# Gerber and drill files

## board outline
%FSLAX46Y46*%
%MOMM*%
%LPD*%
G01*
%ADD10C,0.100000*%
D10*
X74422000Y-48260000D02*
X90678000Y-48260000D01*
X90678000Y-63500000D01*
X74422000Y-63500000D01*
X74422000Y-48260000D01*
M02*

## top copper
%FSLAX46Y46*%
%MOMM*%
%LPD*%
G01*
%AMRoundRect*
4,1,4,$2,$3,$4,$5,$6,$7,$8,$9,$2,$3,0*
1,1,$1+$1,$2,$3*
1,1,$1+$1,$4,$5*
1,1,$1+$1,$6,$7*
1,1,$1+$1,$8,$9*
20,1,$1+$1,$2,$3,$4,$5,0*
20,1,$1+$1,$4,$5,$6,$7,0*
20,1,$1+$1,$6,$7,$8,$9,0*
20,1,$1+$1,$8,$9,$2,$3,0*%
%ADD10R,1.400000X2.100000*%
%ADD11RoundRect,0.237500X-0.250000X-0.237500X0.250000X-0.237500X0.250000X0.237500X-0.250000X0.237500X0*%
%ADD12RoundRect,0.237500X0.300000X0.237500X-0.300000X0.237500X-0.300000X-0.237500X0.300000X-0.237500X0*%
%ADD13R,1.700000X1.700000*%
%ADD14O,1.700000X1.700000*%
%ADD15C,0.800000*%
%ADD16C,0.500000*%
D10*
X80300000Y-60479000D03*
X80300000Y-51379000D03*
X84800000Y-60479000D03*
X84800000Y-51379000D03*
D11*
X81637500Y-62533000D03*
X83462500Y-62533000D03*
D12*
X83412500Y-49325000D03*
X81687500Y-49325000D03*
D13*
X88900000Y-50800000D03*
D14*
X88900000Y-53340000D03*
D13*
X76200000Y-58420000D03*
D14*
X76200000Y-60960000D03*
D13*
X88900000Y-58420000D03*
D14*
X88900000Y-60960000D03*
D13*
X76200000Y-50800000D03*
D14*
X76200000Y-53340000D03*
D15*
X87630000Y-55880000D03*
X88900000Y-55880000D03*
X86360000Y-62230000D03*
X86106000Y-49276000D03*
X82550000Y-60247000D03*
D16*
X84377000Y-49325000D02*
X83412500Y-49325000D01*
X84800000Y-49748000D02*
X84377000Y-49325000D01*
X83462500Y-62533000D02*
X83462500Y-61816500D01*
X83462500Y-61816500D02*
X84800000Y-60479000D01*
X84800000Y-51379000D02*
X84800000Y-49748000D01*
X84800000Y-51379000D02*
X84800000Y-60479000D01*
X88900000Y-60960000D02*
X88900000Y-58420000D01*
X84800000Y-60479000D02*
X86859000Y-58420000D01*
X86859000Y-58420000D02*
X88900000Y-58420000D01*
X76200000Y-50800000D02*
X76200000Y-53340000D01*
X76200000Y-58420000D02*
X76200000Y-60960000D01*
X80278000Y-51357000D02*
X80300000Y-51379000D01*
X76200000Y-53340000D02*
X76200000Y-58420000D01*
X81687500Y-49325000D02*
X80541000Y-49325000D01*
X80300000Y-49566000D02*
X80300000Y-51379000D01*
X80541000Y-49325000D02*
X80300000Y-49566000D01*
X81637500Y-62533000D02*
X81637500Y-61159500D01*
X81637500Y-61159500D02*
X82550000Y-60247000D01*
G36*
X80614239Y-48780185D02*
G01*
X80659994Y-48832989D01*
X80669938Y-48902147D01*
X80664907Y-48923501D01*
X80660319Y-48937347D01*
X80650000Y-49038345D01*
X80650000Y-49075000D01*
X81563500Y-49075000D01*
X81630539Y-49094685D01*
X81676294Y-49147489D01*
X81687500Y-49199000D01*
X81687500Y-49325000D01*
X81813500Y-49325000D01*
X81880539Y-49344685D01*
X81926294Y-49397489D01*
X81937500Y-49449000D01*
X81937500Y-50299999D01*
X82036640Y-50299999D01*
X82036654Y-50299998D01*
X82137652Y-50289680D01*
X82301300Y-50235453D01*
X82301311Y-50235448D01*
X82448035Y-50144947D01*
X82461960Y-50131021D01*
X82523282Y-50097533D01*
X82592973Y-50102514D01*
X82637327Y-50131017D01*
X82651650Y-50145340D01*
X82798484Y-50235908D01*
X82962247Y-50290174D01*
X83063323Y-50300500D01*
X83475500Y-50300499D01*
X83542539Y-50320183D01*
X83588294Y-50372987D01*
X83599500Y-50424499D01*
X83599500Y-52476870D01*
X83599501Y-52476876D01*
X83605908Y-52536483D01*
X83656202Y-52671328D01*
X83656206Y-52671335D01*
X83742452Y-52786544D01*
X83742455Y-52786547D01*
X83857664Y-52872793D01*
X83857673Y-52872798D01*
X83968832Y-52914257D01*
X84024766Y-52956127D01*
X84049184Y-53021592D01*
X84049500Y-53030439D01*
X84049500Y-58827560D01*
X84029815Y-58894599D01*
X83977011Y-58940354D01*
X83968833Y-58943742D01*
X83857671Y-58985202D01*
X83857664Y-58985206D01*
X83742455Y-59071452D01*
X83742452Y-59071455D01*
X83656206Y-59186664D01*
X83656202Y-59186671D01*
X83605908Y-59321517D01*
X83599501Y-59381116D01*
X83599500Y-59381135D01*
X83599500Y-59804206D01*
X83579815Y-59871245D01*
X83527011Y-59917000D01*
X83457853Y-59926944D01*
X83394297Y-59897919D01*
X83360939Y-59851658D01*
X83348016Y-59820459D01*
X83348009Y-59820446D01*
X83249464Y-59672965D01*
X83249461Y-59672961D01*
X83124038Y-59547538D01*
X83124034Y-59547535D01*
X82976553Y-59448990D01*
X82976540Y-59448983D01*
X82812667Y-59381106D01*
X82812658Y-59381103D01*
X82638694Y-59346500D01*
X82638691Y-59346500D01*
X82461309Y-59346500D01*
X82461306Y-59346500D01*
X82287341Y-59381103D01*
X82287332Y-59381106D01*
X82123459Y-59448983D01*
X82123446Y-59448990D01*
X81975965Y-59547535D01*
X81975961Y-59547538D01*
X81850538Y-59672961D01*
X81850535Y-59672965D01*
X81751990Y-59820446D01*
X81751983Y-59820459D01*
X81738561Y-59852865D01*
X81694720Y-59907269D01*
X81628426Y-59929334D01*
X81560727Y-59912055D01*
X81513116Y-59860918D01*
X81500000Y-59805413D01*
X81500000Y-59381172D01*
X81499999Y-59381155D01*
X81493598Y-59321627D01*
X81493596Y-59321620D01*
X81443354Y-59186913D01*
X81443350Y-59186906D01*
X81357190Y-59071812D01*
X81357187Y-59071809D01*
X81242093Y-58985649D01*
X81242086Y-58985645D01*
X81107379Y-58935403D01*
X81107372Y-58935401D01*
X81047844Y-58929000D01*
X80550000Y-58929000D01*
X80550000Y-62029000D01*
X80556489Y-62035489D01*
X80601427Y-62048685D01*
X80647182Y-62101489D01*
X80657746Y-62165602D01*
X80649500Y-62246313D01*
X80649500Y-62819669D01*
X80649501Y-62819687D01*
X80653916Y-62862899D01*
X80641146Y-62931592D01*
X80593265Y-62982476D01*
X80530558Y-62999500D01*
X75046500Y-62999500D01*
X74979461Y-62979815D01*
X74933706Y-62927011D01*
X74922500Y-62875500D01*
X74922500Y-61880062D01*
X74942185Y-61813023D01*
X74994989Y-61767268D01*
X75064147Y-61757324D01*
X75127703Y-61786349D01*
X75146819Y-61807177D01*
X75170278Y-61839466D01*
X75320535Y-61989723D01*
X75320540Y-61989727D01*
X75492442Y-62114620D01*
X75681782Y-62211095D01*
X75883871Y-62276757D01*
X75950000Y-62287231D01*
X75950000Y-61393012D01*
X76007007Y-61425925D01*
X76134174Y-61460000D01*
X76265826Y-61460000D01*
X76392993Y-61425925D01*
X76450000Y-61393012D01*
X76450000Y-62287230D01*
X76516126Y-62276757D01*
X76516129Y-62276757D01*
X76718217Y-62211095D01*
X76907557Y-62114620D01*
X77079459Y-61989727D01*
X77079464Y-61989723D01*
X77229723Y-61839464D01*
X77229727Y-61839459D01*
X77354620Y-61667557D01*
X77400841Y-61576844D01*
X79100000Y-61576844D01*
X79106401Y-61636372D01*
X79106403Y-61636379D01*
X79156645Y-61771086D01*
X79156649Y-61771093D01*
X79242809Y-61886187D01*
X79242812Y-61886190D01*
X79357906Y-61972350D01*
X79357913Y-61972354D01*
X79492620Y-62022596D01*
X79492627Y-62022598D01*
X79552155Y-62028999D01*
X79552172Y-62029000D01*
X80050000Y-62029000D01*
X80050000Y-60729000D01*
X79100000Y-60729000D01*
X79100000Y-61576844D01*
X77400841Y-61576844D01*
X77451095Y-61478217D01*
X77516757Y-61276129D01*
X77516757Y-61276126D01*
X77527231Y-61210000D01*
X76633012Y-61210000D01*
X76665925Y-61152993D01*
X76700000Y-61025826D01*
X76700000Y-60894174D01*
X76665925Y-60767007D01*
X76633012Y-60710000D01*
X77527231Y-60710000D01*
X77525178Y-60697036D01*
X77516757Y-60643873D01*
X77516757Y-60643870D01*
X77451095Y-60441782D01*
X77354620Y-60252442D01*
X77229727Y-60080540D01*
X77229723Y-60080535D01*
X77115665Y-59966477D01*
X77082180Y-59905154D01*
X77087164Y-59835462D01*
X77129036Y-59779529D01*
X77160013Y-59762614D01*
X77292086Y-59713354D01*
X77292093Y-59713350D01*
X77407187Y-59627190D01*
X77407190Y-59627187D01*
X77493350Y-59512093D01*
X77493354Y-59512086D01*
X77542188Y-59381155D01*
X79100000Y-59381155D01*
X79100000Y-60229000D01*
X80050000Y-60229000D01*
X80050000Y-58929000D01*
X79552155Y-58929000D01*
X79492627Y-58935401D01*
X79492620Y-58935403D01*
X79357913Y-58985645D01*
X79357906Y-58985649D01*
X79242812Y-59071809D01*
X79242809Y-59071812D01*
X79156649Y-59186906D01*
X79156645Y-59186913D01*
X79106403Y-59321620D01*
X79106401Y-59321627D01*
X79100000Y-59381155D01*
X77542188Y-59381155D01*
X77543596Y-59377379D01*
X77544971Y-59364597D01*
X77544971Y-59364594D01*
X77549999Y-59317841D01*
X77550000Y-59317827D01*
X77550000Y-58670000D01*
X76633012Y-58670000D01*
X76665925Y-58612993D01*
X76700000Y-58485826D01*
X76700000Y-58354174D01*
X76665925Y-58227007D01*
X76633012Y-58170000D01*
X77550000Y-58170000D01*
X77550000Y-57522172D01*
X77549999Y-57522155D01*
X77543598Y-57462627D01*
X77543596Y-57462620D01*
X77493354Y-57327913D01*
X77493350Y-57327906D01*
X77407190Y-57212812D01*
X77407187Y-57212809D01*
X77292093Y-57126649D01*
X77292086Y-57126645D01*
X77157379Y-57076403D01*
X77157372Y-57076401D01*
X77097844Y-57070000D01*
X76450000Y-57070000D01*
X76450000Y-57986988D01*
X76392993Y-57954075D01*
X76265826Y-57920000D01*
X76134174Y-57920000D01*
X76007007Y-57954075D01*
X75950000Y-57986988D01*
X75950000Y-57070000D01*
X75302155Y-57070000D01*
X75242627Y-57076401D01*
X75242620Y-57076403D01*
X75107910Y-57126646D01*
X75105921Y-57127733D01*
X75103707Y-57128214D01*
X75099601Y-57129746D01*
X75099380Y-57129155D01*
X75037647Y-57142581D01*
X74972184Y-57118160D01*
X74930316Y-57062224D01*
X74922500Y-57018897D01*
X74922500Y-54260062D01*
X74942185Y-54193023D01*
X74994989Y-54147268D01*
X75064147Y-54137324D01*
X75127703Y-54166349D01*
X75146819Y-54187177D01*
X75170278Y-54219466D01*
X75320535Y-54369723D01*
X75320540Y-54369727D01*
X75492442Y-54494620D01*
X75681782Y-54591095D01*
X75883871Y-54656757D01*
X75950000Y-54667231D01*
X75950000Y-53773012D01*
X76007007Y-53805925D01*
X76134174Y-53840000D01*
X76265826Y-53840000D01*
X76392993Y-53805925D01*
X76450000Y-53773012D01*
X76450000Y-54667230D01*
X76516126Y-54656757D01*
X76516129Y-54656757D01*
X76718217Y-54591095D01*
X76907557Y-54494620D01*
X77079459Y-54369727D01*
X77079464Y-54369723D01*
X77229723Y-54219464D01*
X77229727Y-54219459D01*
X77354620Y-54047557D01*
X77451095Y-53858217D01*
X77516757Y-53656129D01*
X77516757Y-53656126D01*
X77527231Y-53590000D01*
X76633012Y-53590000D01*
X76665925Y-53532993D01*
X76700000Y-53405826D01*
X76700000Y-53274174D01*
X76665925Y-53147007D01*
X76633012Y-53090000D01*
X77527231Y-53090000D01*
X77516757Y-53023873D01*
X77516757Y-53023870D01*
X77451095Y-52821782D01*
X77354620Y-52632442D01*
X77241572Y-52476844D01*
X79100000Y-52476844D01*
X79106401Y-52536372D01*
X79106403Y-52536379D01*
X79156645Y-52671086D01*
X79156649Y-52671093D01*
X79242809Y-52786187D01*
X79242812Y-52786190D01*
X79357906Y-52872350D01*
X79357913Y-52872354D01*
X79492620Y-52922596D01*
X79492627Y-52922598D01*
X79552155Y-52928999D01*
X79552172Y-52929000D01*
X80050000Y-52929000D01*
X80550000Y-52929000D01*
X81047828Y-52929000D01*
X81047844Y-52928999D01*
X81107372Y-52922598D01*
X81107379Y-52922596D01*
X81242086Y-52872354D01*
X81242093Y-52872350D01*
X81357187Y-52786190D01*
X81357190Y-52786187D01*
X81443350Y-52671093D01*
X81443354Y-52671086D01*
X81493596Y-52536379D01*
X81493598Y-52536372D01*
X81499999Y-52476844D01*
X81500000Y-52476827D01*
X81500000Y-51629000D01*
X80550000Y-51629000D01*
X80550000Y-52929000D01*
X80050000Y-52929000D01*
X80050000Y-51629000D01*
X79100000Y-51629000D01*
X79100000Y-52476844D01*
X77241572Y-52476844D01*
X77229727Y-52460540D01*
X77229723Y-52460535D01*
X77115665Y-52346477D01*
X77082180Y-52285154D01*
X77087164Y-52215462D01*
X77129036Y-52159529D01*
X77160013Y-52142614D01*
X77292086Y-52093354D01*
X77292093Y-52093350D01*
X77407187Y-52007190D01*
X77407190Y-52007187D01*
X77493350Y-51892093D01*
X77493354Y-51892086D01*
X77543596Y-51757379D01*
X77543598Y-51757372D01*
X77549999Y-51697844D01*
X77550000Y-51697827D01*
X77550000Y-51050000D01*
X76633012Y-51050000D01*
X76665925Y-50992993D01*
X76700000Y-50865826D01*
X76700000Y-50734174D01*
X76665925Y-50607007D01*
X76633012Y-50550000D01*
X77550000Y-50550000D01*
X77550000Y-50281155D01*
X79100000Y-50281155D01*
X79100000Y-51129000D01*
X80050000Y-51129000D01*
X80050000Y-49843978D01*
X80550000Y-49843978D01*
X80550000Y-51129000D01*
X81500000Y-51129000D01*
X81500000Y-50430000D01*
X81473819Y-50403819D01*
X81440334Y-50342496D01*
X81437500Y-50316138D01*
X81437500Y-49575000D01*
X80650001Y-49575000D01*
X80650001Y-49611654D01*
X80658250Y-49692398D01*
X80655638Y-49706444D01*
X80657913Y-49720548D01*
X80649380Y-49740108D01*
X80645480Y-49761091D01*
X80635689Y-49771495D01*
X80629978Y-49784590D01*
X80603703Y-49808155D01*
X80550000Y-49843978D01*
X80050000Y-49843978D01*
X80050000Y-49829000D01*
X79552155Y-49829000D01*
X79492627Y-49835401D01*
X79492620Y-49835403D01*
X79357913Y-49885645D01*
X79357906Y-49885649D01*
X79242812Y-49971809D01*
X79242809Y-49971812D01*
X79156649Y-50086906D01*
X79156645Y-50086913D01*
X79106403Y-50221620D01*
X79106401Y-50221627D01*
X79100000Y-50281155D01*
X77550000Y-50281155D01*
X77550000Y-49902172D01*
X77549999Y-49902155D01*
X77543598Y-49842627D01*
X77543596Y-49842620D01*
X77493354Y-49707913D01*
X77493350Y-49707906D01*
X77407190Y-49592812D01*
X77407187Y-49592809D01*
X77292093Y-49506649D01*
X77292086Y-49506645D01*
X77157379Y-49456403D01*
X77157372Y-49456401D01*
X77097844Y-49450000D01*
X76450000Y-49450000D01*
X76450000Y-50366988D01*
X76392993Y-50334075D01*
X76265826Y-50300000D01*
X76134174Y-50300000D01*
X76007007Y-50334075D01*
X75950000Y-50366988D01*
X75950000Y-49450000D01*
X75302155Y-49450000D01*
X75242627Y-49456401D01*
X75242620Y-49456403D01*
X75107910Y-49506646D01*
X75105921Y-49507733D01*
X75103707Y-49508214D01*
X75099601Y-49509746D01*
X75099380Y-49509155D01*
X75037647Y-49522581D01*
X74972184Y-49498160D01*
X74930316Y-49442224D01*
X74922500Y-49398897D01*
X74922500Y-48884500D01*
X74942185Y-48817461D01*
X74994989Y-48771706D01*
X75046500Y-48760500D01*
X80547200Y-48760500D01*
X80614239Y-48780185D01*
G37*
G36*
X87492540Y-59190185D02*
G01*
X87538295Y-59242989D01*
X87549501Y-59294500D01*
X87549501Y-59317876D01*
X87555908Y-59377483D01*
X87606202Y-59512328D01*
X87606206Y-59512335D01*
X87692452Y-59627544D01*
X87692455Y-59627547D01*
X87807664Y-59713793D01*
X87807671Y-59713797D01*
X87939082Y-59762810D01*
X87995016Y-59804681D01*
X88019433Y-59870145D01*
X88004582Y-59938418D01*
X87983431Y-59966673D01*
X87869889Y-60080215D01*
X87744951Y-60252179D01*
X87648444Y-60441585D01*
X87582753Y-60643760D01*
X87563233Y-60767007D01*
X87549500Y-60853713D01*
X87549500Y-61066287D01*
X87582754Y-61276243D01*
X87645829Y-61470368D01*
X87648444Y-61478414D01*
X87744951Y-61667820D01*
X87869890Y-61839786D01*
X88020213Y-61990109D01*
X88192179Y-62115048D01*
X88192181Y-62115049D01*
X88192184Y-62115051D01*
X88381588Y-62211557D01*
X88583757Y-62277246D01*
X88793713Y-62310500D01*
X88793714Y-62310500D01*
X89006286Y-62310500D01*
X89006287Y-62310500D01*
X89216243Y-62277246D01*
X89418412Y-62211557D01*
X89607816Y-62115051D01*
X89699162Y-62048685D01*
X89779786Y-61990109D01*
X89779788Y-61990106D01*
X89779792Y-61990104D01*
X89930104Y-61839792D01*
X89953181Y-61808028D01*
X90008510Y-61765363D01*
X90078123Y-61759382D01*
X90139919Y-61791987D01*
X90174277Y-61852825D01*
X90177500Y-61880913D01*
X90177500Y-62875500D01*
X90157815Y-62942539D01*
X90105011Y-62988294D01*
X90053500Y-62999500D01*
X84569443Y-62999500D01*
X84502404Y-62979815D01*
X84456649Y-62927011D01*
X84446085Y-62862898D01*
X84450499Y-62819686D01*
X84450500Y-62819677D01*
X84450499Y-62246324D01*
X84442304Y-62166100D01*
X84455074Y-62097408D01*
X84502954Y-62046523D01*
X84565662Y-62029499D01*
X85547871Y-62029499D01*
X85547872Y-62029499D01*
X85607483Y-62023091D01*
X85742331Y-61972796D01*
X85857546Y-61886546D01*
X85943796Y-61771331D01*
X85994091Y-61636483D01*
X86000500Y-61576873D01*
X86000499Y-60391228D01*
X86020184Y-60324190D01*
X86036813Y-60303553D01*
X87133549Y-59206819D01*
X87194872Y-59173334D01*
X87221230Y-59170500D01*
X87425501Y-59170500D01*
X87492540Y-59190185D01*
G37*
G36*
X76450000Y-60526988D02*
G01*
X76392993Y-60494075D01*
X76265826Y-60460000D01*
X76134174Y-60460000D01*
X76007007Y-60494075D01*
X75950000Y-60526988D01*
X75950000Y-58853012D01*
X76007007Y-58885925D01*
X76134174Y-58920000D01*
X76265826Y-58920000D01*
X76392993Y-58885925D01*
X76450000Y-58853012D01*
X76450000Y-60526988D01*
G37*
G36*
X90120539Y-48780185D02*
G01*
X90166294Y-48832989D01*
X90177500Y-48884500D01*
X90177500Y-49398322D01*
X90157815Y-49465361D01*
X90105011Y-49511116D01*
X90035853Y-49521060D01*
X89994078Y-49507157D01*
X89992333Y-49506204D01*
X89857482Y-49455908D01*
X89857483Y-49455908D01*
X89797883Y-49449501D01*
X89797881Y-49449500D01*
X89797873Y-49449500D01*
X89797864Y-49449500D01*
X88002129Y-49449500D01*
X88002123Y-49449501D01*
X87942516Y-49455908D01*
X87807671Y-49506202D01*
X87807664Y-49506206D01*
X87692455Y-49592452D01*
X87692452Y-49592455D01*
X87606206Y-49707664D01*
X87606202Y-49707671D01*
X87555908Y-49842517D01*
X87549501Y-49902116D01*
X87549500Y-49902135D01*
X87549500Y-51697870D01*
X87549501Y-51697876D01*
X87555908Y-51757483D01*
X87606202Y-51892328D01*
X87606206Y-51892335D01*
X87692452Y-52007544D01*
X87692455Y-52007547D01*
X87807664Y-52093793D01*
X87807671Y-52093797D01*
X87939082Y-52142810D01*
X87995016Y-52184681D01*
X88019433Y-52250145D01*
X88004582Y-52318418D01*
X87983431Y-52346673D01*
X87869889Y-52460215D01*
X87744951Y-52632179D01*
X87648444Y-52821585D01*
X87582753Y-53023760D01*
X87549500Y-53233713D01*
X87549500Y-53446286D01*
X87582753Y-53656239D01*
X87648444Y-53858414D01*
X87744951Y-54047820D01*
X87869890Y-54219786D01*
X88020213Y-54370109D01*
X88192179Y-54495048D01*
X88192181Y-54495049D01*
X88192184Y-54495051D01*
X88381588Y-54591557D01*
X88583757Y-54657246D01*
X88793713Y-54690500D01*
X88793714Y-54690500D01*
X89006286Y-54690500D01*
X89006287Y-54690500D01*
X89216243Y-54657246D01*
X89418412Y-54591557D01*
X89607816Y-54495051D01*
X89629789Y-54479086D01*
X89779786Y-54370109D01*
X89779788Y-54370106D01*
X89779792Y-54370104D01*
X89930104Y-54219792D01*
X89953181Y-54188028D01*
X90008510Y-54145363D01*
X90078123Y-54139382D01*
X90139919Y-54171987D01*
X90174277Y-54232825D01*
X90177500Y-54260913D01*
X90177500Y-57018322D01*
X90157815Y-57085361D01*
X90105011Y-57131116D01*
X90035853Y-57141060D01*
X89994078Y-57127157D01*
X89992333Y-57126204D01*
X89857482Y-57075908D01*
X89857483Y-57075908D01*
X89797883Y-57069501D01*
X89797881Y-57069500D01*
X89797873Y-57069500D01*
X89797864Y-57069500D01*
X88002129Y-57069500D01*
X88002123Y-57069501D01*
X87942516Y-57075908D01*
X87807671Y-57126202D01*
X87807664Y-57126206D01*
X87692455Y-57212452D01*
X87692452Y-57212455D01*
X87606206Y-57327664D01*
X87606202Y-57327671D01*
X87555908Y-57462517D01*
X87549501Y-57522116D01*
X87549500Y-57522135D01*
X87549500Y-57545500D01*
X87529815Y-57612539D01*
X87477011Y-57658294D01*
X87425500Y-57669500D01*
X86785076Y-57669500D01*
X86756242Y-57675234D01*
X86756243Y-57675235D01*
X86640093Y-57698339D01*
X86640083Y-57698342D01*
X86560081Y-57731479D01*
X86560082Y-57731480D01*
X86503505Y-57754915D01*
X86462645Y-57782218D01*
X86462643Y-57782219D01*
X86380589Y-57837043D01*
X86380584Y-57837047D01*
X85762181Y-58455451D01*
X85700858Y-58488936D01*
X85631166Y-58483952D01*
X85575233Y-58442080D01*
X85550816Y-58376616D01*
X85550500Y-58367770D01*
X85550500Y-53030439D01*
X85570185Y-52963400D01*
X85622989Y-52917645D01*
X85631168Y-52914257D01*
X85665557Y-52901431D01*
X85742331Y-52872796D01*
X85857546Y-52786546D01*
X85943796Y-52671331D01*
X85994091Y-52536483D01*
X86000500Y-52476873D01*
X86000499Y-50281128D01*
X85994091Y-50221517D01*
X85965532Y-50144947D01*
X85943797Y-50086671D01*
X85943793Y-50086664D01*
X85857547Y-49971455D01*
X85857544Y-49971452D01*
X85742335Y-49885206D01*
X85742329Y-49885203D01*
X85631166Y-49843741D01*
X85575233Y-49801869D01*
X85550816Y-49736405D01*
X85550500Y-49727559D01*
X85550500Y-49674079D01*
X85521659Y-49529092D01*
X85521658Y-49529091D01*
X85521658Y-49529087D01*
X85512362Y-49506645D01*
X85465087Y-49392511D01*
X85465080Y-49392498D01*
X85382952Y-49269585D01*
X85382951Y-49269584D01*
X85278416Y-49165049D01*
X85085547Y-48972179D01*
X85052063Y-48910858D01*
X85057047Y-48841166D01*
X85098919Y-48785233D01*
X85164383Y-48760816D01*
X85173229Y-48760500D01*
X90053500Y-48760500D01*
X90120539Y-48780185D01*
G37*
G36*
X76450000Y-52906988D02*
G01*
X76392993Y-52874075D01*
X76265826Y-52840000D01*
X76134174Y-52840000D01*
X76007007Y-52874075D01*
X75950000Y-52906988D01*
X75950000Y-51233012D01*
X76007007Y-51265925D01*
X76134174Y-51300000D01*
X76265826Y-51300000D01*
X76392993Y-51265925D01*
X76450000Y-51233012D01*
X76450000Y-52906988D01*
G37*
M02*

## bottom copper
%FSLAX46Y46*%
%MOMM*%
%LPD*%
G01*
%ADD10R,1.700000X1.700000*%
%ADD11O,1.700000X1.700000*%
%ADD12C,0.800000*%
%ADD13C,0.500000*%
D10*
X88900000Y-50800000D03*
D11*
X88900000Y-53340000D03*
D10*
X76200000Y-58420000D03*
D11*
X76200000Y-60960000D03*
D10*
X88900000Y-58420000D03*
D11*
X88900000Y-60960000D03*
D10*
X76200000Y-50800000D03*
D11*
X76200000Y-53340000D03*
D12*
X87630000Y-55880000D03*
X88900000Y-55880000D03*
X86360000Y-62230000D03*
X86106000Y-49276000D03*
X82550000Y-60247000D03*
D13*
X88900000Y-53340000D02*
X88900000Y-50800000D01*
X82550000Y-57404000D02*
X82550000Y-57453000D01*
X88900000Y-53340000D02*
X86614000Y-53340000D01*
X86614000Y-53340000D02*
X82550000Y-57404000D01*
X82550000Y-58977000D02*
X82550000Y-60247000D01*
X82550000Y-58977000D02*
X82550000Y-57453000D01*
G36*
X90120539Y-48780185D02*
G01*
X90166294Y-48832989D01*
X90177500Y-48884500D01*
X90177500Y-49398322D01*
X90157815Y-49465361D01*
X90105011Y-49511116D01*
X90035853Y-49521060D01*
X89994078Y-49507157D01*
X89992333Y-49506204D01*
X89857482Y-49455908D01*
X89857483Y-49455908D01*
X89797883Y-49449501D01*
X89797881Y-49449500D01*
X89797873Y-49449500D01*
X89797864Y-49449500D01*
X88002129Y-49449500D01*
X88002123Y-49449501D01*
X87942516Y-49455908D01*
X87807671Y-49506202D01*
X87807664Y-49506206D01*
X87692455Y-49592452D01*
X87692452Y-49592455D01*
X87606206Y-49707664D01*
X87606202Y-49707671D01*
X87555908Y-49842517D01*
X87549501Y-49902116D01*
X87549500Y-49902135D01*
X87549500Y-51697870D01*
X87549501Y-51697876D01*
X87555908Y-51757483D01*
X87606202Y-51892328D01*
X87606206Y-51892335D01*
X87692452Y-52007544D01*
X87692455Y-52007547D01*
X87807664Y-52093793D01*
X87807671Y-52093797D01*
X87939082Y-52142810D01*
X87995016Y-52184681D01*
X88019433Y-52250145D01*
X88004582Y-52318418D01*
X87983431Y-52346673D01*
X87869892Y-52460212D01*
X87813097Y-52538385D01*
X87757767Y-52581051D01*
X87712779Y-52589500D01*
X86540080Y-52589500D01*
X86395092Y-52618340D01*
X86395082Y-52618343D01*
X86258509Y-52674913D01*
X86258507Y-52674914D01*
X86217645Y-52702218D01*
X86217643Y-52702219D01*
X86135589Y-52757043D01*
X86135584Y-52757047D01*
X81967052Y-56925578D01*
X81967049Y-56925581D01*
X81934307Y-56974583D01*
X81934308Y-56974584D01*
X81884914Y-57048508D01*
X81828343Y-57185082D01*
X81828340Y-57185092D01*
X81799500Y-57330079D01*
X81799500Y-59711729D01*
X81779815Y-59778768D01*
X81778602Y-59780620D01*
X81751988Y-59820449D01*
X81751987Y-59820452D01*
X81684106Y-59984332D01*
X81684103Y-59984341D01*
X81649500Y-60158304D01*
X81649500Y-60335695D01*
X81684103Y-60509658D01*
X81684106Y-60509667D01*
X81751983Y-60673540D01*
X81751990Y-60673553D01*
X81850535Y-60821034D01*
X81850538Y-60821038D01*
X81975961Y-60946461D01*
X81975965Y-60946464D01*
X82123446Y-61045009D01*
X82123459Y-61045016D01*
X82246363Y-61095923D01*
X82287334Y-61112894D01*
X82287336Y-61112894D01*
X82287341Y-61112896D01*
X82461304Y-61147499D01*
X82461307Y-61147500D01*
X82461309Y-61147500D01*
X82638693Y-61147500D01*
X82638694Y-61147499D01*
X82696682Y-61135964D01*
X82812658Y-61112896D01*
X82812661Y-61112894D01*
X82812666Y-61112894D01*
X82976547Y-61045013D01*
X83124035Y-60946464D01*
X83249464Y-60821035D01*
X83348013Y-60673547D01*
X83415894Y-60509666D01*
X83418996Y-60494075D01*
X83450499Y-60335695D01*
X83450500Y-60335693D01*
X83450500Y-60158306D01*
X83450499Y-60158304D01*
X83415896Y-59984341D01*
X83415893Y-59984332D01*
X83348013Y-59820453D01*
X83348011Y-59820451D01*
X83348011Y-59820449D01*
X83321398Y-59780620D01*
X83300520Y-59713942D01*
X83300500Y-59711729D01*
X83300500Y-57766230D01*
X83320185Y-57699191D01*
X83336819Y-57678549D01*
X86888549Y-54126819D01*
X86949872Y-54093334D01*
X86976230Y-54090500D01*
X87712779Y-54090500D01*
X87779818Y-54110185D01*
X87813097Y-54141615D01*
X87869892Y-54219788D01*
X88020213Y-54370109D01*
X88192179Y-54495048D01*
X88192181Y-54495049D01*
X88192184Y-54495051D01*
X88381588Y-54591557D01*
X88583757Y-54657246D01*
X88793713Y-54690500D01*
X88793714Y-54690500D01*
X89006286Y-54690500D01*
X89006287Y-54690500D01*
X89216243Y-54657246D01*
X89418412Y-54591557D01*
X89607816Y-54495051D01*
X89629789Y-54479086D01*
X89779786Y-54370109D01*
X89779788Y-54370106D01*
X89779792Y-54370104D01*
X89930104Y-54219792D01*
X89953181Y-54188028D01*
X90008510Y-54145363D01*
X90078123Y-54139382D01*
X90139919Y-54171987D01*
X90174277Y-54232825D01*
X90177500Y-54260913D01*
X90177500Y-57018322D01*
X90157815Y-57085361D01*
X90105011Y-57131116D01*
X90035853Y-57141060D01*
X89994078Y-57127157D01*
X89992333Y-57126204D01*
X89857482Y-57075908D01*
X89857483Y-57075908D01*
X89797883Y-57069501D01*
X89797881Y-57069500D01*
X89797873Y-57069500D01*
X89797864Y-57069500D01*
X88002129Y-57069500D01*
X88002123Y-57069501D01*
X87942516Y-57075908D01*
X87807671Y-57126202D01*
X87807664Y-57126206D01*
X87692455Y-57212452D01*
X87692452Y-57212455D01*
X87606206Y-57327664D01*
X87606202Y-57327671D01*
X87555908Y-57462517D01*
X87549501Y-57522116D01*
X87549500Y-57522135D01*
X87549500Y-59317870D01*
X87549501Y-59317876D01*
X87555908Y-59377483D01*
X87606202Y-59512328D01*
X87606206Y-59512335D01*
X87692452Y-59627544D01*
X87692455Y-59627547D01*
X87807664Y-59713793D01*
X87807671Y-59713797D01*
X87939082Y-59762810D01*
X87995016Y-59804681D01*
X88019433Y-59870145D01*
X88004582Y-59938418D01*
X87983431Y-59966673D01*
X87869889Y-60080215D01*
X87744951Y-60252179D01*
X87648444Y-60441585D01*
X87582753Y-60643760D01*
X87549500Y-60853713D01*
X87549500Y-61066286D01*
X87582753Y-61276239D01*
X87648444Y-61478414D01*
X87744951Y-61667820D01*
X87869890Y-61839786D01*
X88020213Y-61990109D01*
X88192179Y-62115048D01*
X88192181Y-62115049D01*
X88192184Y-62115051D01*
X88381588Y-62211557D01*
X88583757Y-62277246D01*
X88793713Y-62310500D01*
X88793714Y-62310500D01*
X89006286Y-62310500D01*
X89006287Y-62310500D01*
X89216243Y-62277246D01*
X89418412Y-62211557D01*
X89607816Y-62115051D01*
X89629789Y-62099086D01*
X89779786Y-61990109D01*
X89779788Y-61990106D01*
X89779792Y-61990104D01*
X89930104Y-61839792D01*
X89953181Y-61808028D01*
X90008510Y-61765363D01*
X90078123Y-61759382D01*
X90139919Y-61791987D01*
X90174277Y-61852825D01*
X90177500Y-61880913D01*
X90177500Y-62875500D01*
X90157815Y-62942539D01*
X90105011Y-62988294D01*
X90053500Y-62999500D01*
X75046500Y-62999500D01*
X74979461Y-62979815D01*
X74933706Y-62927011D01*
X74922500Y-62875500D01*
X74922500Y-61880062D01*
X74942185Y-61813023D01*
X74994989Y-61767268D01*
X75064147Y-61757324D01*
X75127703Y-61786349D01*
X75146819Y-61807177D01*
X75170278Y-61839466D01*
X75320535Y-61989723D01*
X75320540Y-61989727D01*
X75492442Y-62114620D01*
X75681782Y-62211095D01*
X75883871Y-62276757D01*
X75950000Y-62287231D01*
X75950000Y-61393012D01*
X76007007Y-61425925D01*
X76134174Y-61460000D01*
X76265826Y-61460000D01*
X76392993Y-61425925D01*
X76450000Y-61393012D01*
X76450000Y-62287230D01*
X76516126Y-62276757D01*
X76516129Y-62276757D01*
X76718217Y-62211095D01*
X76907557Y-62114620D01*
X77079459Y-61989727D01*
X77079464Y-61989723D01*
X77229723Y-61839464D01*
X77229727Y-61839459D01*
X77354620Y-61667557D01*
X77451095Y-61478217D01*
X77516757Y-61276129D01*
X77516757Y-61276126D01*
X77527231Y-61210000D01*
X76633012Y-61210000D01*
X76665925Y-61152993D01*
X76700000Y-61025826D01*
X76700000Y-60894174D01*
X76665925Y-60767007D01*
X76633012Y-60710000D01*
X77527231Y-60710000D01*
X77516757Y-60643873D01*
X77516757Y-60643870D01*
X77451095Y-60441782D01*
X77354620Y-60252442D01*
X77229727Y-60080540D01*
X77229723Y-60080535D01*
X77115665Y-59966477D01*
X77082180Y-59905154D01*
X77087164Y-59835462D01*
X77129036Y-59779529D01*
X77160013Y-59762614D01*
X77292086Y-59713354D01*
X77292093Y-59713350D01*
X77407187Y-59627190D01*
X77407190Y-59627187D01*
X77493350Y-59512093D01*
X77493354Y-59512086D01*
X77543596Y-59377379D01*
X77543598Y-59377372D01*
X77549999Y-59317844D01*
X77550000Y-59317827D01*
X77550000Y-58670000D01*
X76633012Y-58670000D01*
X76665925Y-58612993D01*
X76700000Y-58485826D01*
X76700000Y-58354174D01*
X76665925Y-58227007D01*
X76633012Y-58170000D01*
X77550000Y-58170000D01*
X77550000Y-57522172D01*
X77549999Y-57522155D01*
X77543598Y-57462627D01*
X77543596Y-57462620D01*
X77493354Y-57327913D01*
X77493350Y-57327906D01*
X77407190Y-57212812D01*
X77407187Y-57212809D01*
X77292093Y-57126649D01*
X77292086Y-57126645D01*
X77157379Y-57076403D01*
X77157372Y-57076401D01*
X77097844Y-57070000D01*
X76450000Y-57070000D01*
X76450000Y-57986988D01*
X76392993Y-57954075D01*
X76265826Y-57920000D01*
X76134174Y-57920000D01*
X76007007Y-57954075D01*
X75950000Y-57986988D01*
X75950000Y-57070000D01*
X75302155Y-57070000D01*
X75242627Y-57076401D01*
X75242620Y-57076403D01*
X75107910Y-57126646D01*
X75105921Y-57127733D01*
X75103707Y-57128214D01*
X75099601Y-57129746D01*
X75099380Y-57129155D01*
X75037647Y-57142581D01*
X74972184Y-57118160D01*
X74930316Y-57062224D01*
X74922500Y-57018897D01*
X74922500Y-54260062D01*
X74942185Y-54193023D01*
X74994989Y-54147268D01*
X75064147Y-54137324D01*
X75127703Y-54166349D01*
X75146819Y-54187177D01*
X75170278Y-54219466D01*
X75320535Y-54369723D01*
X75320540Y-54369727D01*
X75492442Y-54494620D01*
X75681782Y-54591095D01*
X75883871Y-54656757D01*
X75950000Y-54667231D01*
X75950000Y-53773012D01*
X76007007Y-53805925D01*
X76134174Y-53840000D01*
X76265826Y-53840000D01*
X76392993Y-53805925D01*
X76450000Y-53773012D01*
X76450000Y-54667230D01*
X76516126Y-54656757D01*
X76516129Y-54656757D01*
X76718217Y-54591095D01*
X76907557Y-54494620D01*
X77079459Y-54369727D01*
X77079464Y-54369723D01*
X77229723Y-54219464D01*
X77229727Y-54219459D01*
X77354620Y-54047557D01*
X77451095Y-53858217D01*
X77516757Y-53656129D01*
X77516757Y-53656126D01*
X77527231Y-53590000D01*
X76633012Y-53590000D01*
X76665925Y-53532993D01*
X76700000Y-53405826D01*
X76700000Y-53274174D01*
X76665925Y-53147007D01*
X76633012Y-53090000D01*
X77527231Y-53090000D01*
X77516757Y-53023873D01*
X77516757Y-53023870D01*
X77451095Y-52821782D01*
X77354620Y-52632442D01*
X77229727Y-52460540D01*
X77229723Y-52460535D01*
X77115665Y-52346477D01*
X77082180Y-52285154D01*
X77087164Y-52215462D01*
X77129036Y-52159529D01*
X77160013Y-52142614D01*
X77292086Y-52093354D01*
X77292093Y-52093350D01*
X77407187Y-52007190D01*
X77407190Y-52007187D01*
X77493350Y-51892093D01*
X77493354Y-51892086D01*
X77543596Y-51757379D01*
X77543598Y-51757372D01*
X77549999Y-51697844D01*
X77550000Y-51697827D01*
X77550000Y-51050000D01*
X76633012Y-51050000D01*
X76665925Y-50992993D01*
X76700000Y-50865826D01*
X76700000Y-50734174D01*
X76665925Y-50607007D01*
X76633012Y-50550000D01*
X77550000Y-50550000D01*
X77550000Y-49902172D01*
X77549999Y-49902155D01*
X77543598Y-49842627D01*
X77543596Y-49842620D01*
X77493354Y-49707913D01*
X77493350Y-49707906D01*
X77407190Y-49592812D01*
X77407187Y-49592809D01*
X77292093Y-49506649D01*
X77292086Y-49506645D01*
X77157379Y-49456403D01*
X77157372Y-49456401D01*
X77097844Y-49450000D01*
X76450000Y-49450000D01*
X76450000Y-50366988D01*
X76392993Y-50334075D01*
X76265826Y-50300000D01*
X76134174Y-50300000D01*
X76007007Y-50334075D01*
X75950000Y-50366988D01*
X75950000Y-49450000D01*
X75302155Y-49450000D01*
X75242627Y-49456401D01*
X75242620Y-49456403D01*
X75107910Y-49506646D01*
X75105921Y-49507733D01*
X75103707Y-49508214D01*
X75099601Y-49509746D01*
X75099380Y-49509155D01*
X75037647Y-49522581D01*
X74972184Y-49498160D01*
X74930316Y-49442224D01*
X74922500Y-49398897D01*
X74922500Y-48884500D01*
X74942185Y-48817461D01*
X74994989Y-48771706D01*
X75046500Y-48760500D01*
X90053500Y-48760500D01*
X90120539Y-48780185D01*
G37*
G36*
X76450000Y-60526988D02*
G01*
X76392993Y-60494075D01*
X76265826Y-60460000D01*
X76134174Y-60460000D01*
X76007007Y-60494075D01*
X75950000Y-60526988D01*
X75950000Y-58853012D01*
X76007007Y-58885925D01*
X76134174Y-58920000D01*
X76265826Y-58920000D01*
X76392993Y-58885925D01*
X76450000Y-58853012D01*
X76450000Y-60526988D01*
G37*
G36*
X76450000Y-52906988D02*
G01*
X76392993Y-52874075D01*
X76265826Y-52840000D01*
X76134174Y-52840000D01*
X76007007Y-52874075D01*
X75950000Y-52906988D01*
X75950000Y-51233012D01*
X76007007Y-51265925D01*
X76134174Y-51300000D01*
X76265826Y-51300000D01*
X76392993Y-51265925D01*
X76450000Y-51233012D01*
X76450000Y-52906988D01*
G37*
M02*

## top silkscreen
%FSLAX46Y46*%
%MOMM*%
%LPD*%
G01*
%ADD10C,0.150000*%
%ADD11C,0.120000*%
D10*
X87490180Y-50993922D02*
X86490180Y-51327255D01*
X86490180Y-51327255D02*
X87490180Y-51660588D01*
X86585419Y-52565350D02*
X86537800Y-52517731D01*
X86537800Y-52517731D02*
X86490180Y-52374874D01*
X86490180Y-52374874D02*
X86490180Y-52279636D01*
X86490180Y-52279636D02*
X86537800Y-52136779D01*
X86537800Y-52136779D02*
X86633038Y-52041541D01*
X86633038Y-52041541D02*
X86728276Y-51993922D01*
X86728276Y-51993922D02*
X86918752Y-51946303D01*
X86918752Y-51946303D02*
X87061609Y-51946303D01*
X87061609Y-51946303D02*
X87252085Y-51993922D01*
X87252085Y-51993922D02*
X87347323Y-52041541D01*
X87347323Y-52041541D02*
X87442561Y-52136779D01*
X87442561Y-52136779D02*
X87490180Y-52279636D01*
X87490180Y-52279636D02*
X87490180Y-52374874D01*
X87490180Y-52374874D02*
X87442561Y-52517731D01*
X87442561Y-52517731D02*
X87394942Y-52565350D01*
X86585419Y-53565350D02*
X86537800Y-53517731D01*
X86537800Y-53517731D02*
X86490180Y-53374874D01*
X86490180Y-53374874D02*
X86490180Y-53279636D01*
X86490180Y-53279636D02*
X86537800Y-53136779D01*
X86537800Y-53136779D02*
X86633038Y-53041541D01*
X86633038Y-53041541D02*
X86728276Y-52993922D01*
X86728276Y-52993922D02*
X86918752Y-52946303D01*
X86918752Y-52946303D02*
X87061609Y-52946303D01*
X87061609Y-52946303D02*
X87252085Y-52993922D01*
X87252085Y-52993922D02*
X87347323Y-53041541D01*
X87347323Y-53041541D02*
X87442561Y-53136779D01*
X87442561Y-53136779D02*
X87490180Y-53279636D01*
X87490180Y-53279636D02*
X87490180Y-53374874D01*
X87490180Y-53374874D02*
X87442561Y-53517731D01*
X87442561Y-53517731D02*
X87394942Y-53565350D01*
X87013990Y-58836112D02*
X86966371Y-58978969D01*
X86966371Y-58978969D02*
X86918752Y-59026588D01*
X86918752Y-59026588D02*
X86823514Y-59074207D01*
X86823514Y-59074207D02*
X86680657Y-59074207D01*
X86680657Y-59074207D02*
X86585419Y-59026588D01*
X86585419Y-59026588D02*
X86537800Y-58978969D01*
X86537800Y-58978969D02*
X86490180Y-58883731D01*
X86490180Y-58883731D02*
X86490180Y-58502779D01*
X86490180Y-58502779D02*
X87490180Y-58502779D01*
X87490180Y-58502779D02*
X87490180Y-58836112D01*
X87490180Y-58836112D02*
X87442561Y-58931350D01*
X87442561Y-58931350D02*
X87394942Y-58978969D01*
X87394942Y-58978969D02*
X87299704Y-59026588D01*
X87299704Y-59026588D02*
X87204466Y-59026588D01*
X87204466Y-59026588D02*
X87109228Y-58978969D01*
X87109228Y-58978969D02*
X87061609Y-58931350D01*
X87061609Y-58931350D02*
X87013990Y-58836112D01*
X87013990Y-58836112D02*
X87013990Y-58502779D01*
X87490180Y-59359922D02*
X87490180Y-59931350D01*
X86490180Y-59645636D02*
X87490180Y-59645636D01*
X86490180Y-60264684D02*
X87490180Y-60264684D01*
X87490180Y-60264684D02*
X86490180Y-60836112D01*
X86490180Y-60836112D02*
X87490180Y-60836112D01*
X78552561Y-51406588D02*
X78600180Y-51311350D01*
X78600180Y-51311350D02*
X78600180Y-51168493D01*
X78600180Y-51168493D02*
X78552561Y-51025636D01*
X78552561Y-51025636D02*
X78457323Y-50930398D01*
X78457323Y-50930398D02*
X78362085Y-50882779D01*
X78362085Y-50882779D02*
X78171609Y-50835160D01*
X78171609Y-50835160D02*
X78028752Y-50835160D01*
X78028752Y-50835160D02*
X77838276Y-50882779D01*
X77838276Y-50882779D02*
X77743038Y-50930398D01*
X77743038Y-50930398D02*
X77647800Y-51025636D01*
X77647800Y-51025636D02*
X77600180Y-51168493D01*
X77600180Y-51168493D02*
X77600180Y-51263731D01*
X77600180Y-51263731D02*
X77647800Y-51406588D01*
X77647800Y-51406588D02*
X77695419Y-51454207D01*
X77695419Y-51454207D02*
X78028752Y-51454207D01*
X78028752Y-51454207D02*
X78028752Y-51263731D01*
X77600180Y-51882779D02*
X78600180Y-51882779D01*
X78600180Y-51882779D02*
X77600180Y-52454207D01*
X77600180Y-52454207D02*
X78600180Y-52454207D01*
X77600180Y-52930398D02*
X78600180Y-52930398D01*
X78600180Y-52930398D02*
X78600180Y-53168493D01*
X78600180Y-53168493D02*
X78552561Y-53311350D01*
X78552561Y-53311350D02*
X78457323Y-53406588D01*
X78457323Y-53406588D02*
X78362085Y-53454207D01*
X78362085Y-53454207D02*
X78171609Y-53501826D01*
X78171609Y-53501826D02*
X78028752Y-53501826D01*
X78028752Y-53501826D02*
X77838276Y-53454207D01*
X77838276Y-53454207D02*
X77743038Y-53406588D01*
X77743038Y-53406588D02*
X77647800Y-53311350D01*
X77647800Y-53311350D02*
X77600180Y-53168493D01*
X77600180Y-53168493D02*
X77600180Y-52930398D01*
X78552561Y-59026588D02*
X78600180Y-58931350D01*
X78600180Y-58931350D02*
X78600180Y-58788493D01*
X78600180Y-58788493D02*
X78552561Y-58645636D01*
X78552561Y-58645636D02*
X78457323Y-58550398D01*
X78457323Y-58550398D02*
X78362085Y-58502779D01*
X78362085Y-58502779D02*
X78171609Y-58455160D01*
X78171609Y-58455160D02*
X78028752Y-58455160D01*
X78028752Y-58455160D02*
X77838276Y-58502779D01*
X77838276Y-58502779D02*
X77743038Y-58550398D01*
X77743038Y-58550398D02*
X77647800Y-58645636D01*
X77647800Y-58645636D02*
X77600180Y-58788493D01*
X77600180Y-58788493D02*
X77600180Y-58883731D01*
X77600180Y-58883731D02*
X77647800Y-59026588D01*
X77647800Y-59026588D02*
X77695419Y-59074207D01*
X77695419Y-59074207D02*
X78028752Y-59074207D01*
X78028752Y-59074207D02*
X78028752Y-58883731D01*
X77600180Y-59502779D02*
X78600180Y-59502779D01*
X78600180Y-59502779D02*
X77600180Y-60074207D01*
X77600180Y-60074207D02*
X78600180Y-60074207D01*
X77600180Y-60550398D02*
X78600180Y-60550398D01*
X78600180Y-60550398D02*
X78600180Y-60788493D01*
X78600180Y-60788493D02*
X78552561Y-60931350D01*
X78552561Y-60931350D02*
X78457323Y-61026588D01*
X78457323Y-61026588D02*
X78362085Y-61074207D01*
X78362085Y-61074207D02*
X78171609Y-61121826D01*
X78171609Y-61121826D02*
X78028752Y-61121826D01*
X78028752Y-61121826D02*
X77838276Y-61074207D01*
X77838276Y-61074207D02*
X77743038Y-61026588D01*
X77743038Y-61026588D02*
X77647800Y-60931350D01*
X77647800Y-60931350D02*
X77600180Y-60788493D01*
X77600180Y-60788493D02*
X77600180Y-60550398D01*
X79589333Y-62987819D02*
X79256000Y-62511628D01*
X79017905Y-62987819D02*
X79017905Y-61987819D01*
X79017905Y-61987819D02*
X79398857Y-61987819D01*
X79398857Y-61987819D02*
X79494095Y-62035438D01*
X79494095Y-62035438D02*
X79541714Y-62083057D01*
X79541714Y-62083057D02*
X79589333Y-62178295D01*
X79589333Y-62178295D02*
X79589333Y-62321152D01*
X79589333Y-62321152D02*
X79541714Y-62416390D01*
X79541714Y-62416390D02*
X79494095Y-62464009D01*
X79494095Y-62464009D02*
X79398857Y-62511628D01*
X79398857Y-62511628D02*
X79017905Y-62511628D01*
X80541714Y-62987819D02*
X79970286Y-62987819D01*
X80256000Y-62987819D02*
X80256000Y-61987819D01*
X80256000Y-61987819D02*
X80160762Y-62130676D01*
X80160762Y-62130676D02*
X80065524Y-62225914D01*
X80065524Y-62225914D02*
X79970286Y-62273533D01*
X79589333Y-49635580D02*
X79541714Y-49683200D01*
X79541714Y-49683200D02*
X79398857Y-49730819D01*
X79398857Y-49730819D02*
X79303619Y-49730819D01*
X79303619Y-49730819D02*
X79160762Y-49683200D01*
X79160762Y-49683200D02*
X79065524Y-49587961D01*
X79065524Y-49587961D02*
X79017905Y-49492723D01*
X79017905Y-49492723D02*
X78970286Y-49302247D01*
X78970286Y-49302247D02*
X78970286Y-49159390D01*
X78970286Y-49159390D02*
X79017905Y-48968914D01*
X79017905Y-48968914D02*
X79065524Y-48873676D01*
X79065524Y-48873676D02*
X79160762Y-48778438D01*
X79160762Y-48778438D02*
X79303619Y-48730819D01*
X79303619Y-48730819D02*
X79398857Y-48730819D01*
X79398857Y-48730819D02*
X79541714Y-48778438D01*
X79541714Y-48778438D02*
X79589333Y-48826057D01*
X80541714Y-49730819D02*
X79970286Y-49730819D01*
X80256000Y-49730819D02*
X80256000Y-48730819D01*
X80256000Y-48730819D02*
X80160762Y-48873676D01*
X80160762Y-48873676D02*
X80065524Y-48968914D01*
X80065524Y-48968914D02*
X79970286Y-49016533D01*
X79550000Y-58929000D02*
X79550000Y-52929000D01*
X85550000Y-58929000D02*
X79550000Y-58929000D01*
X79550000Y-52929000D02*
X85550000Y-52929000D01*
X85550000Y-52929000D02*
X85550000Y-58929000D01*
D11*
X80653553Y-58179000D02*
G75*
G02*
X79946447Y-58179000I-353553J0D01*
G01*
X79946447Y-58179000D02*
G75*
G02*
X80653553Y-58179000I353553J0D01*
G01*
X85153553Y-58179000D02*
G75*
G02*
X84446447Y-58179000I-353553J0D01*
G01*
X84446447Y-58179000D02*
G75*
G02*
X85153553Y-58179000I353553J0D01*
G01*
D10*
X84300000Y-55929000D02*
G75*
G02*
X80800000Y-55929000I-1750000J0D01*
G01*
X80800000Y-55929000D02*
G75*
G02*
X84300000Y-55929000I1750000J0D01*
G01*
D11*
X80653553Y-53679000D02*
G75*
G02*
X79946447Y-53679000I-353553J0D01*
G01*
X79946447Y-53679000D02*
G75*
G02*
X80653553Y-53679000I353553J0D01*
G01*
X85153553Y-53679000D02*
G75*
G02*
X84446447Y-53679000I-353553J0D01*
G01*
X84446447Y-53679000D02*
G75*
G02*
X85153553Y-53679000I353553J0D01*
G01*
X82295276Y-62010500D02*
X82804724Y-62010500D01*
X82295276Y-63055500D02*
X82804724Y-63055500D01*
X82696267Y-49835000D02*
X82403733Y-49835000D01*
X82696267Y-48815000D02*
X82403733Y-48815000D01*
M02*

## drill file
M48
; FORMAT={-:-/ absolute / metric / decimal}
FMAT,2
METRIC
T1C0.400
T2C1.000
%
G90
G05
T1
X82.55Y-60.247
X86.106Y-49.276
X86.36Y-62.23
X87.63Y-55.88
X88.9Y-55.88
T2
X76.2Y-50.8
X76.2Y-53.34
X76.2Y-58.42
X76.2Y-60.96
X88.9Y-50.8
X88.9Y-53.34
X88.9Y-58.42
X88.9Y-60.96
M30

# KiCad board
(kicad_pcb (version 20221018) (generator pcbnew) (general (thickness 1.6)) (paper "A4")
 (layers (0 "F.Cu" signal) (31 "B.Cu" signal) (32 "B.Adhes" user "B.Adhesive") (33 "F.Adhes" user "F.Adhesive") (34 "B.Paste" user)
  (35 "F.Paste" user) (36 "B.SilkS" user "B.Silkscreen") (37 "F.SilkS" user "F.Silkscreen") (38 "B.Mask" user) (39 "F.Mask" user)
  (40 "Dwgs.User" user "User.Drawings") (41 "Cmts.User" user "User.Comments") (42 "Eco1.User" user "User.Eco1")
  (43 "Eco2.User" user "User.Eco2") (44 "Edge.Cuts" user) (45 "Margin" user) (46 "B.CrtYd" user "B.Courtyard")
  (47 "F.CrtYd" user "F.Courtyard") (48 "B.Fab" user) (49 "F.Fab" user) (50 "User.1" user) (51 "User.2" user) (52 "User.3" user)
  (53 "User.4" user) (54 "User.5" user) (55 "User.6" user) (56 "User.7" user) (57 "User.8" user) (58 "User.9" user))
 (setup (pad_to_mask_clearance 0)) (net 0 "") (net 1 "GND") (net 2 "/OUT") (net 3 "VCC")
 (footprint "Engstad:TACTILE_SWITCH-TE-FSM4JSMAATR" (layer "F.Cu") (at 82.55 55.929 90)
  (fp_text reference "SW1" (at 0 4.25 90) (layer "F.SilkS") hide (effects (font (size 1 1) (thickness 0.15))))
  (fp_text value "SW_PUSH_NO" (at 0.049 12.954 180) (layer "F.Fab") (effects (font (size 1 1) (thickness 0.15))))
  (fp_line (start -3 -3) (end 3 -3) (stroke (width 0.15) (type solid)) (layer "F.SilkS"))
  (fp_line (start -3 3) (end -3 -3) (stroke (width 0.15) (type solid)) (layer "F.SilkS"))
  (fp_line (start 3 -3) (end 3 3) (stroke (width 0.15) (type solid)) (layer "F.SilkS"))
  (fp_line (start 3 3) (end -3 3) (stroke (width 0.15) (type solid)) (layer "F.SilkS"))
  (fp_circle (center -2.25 -2.25) (end -2 -2) (stroke (width 0.12) (type solid)) (fill none) (layer "F.SilkS"))
  (fp_circle (center -2.25 2.25) (end -2.5 2.5) (stroke (width 0.12) (type solid)) (fill none) (layer "F.SilkS"))
  (fp_circle (center 0 0) (end 1.75 0) (stroke (width 0.15) (type solid)) (fill none) (layer "F.SilkS"))
  (fp_circle (center 2.25 -2.25) (end 2 -2.5) (stroke (width 0.12) (type solid)) (fill none) (layer "F.SilkS"))
  (fp_circle (center 2.25 2.25) (end 2.5 2.5) (stroke (width 0.12) (type solid)) (fill none) (layer "F.SilkS"))
  (pad "1" smd rect (at -4.55 -2.25 90) (size 2.1 1.4) (layers "F.Cu" "F.Paste" "F.Mask") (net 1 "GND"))
  (pad "1" smd rect (at 4.55 -2.25 270) (size 2.1 1.4) (layers "F.Cu" "F.Paste" "F.Mask") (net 1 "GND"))
  (pad "2" smd rect (at -4.55 2.25 270) (size 2.1 1.4) (layers "F.Cu" "F.Paste" "F.Mask") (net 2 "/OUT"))
  (pad "2" smd rect (at 4.55 2.25 270) (size 2.1 1.4) (layers "F.Cu" "F.Paste" "F.Mask") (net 2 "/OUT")))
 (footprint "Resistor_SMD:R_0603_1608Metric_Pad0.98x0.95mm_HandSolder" (layer "F.Cu") (at 82.55 62.533)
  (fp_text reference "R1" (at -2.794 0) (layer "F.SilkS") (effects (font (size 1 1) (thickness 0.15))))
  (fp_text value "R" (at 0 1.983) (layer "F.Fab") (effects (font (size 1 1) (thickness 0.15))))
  (fp_line (start -0.254724 -0.5225) (end 0.254724 -0.5225) (stroke (width 0.12) (type solid)) (layer "F.SilkS"))
  (fp_line (start -0.254724 0.5225) (end 0.254724 0.5225) (stroke (width 0.12) (type solid)) (layer "F.SilkS"))
  (pad "1" smd roundrect (at -0.9125 0) (size 0.975 0.95) (layers "F.Cu" "F.Paste" "F.Mask") (roundrect_rratio 0.25) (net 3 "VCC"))
  (pad "2" smd roundrect (at 0.9125 0) (size 0.975 0.95) (layers "F.Cu" "F.Paste" "F.Mask") (roundrect_rratio 0.25) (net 2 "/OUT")))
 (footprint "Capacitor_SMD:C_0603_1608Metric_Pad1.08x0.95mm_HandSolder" (layer "F.Cu") (at 82.55 49.325 180)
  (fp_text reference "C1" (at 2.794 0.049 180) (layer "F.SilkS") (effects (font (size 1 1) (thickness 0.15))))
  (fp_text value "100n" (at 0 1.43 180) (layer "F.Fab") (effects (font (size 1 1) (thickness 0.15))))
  (fp_line (start -0.146267 -0.51) (end 0.146267 -0.51) (stroke (width 0.12) (type solid)) (layer "F.SilkS"))
  (fp_line (start -0.146267 0.51) (end 0.146267 0.51) (stroke (width 0.12) (type solid)) (layer "F.SilkS"))
  (pad "1" smd roundrect (at -0.8625 0 180) (size 1.075 0.95) (layers "F.Cu" "F.Paste" "F.Mask") (roundrect_rratio 0.25) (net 2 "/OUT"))
  (pad "2" smd roundrect (at 0.8625 0 180) (size 1.075 0.95) (layers "F.Cu" "F.Paste" "F.Mask") (roundrect_rratio 0.25) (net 1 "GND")))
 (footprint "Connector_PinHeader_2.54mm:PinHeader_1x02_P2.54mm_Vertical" (layer "B.Cu") (at 88.9 50.8 180)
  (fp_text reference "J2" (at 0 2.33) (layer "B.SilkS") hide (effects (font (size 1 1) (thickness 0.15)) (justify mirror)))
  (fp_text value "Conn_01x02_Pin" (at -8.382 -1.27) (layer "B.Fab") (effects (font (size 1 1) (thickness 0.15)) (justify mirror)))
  (pad "1" thru_hole rect (at 0 0 180) (size 1.7 1.7) (drill 1) (layers "*.Cu" "*.Mask") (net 3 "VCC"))
  (pad "2" thru_hole oval (at 0 -2.54 180) (size 1.7 1.7) (drill 1) (layers "*.Cu" "*.Mask") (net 3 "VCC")))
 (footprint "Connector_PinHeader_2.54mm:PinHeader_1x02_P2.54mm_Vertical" (layer "B.Cu") (at 76.2 58.42 180)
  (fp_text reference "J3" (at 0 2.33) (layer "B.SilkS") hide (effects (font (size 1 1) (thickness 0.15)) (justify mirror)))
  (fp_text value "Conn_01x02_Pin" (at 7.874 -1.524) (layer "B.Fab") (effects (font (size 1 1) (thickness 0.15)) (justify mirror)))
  (pad "1" thru_hole rect (at 0 0 180) (size 1.7 1.7) (drill 1) (layers "*.Cu" "*.Mask") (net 1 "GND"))
  (pad "2" thru_hole oval (at 0 -2.54 180) (size 1.7 1.7) (drill 1) (layers "*.Cu" "*.Mask") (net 1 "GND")))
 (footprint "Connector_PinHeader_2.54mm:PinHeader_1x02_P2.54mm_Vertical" (layer "B.Cu") (at 88.9 58.42 180)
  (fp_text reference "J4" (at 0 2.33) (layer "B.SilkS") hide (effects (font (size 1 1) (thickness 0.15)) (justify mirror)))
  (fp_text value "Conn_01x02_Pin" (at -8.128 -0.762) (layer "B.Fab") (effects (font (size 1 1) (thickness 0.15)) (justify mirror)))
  (pad "1" thru_hole rect (at 0 0 180) (size 1.7 1.7) (drill 1) (layers "*.Cu" "*.Mask") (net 2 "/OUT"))
  (pad "2" thru_hole oval (at 0 -2.54 180) (size 1.7 1.7) (drill 1) (layers "*.Cu" "*.Mask") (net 2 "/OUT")))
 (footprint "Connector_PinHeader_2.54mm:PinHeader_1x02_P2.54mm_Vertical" (layer "B.Cu") (at 76.2 50.8 180)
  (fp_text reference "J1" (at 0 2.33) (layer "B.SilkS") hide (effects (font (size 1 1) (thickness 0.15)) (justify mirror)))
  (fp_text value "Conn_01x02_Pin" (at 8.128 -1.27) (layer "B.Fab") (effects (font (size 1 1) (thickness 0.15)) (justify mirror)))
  (pad "1" thru_hole rect (at 0 0 180) (size 1.7 1.7) (drill 1) (layers "*.Cu" "*.Mask") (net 1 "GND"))
  (pad "2" thru_hole oval (at 0 -2.54 180) (size 1.7 1.7) (drill 1) (layers "*.Cu" "*.Mask") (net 1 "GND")))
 (gr_rect (start 74.422 48.26) (end 90.678 63.5) (stroke (width 0.1) (type default)) (fill none) (layer "Edge.Cuts"))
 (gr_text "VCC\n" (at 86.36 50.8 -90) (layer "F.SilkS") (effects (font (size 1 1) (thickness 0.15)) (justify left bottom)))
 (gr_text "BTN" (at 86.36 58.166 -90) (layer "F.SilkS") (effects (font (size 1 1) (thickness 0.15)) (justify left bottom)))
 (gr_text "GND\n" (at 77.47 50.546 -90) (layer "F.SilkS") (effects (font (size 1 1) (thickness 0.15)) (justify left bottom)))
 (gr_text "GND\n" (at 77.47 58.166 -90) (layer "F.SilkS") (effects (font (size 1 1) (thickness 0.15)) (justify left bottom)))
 (segment (start 84.377 49.325) (end 83.4125 49.325) (width 0.5) (layer "F.Cu") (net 2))
 (segment (start 84.8 49.748) (end 84.377 49.325) (width 0.5) (layer "F.Cu") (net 2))
 (segment (start 83.4625 62.533) (end 83.4625 61.8165) (width 0.5) (layer "F.Cu") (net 2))
 (segment (start 83.4625 61.8165) (end 84.8 60.479) (width 0.5) (layer "F.Cu") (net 2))
 (segment (start 84.8 51.379) (end 84.8 49.748) (width 0.5) (layer "F.Cu") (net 2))
 (segment (start 84.8 51.379) (end 84.8 60.479) (width 0.5) (layer "F.Cu") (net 2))
 (segment (start 88.9 60.96) (end 88.9 58.42) (width 0.5) (layer "F.Cu") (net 2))
 (segment (start 84.8 60.479) (end 86.859 58.42) (width 0.5) (layer "F.Cu") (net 2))
 (segment (start 86.859 58.42) (end 88.9 58.42) (width 0.5) (layer "F.Cu") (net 2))
 (segment (start 76.2 50.8) (end 76.2 53.34) (width 0.5) (layer "F.Cu") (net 1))
 (segment (start 76.2 58.42) (end 76.2 60.96) (width 0.5) (layer "F.Cu") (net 1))
 (segment (start 80.278 51.357) (end 80.3 51.379) (width 0.5) (layer "F.Cu") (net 1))
 (segment (start 76.2 53.34) (end 76.2 58.42) (width 0.5) (layer "F.Cu") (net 1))
 (segment (start 81.6875 49.325) (end 80.541 49.325) (width 0.5) (layer "F.Cu") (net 1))
 (segment (start 80.3 49.566) (end 80.3 51.379) (width 0.5) (layer "F.Cu") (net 1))
 (segment (start 80.541 49.325) (end 80.3 49.566) (width 0.5) (layer "F.Cu") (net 1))
 (via (at 87.63 55.88) (size 0.8) (drill 0.4) (layers "F.Cu" "B.Cu") (free) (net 1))
 (via (at 88.9 55.88) (size 0.8) (drill 0.4) (layers "F.Cu" "B.Cu") (free) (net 1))
 (via (at 86.36 62.23) (size 0.8) (drill 0.4) (layers "F.Cu" "B.Cu") (free) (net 1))
 (via (at 86.106 49.276) (size 0.8) (drill 0.4) (layers "F.Cu" "B.Cu") (free) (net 1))
 (segment (start 81.6375 62.533) (end 81.6375 61.1595) (width 0.5) (layer "F.Cu") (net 3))
 (segment (start 81.6375 61.1595) (end 82.55 60.247) (width 0.5) (layer "F.Cu") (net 3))
 (via (at 82.55 60.247) (size 0.8) (drill 0.4) (layers "F.Cu" "B.Cu") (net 3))
 (segment (start 88.9 53.34) (end 88.9 50.8) (width 0.5) (layer "B.Cu") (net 3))
 (segment (start 82.55 57.404) (end 82.55 57.453) (width 0.5) (layer "B.Cu") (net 3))
 (segment (start 88.9 53.34) (end 86.614 53.34) (width 0.5) (layer "B.Cu") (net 3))
 (segment (start 86.614 53.34) (end 82.55 57.404) (width 0.5) (layer "B.Cu") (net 3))
 (segment (start 82.55 58.977) (end 82.55 60.247) (width 0.5) (layer "B.Cu") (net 3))
 (segment (start 82.55 58.977) (end 82.55 57.453) (width 0.5) (layer "B.Cu") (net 3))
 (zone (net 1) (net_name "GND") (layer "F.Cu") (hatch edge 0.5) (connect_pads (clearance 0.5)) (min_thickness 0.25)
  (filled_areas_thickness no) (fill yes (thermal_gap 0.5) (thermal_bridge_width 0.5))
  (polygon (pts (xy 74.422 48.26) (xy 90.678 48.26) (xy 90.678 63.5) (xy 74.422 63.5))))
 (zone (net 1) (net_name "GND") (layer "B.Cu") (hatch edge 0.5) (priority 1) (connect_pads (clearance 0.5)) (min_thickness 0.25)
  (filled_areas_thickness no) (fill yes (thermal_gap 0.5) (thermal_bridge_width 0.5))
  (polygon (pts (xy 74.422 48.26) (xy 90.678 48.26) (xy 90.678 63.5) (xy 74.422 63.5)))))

